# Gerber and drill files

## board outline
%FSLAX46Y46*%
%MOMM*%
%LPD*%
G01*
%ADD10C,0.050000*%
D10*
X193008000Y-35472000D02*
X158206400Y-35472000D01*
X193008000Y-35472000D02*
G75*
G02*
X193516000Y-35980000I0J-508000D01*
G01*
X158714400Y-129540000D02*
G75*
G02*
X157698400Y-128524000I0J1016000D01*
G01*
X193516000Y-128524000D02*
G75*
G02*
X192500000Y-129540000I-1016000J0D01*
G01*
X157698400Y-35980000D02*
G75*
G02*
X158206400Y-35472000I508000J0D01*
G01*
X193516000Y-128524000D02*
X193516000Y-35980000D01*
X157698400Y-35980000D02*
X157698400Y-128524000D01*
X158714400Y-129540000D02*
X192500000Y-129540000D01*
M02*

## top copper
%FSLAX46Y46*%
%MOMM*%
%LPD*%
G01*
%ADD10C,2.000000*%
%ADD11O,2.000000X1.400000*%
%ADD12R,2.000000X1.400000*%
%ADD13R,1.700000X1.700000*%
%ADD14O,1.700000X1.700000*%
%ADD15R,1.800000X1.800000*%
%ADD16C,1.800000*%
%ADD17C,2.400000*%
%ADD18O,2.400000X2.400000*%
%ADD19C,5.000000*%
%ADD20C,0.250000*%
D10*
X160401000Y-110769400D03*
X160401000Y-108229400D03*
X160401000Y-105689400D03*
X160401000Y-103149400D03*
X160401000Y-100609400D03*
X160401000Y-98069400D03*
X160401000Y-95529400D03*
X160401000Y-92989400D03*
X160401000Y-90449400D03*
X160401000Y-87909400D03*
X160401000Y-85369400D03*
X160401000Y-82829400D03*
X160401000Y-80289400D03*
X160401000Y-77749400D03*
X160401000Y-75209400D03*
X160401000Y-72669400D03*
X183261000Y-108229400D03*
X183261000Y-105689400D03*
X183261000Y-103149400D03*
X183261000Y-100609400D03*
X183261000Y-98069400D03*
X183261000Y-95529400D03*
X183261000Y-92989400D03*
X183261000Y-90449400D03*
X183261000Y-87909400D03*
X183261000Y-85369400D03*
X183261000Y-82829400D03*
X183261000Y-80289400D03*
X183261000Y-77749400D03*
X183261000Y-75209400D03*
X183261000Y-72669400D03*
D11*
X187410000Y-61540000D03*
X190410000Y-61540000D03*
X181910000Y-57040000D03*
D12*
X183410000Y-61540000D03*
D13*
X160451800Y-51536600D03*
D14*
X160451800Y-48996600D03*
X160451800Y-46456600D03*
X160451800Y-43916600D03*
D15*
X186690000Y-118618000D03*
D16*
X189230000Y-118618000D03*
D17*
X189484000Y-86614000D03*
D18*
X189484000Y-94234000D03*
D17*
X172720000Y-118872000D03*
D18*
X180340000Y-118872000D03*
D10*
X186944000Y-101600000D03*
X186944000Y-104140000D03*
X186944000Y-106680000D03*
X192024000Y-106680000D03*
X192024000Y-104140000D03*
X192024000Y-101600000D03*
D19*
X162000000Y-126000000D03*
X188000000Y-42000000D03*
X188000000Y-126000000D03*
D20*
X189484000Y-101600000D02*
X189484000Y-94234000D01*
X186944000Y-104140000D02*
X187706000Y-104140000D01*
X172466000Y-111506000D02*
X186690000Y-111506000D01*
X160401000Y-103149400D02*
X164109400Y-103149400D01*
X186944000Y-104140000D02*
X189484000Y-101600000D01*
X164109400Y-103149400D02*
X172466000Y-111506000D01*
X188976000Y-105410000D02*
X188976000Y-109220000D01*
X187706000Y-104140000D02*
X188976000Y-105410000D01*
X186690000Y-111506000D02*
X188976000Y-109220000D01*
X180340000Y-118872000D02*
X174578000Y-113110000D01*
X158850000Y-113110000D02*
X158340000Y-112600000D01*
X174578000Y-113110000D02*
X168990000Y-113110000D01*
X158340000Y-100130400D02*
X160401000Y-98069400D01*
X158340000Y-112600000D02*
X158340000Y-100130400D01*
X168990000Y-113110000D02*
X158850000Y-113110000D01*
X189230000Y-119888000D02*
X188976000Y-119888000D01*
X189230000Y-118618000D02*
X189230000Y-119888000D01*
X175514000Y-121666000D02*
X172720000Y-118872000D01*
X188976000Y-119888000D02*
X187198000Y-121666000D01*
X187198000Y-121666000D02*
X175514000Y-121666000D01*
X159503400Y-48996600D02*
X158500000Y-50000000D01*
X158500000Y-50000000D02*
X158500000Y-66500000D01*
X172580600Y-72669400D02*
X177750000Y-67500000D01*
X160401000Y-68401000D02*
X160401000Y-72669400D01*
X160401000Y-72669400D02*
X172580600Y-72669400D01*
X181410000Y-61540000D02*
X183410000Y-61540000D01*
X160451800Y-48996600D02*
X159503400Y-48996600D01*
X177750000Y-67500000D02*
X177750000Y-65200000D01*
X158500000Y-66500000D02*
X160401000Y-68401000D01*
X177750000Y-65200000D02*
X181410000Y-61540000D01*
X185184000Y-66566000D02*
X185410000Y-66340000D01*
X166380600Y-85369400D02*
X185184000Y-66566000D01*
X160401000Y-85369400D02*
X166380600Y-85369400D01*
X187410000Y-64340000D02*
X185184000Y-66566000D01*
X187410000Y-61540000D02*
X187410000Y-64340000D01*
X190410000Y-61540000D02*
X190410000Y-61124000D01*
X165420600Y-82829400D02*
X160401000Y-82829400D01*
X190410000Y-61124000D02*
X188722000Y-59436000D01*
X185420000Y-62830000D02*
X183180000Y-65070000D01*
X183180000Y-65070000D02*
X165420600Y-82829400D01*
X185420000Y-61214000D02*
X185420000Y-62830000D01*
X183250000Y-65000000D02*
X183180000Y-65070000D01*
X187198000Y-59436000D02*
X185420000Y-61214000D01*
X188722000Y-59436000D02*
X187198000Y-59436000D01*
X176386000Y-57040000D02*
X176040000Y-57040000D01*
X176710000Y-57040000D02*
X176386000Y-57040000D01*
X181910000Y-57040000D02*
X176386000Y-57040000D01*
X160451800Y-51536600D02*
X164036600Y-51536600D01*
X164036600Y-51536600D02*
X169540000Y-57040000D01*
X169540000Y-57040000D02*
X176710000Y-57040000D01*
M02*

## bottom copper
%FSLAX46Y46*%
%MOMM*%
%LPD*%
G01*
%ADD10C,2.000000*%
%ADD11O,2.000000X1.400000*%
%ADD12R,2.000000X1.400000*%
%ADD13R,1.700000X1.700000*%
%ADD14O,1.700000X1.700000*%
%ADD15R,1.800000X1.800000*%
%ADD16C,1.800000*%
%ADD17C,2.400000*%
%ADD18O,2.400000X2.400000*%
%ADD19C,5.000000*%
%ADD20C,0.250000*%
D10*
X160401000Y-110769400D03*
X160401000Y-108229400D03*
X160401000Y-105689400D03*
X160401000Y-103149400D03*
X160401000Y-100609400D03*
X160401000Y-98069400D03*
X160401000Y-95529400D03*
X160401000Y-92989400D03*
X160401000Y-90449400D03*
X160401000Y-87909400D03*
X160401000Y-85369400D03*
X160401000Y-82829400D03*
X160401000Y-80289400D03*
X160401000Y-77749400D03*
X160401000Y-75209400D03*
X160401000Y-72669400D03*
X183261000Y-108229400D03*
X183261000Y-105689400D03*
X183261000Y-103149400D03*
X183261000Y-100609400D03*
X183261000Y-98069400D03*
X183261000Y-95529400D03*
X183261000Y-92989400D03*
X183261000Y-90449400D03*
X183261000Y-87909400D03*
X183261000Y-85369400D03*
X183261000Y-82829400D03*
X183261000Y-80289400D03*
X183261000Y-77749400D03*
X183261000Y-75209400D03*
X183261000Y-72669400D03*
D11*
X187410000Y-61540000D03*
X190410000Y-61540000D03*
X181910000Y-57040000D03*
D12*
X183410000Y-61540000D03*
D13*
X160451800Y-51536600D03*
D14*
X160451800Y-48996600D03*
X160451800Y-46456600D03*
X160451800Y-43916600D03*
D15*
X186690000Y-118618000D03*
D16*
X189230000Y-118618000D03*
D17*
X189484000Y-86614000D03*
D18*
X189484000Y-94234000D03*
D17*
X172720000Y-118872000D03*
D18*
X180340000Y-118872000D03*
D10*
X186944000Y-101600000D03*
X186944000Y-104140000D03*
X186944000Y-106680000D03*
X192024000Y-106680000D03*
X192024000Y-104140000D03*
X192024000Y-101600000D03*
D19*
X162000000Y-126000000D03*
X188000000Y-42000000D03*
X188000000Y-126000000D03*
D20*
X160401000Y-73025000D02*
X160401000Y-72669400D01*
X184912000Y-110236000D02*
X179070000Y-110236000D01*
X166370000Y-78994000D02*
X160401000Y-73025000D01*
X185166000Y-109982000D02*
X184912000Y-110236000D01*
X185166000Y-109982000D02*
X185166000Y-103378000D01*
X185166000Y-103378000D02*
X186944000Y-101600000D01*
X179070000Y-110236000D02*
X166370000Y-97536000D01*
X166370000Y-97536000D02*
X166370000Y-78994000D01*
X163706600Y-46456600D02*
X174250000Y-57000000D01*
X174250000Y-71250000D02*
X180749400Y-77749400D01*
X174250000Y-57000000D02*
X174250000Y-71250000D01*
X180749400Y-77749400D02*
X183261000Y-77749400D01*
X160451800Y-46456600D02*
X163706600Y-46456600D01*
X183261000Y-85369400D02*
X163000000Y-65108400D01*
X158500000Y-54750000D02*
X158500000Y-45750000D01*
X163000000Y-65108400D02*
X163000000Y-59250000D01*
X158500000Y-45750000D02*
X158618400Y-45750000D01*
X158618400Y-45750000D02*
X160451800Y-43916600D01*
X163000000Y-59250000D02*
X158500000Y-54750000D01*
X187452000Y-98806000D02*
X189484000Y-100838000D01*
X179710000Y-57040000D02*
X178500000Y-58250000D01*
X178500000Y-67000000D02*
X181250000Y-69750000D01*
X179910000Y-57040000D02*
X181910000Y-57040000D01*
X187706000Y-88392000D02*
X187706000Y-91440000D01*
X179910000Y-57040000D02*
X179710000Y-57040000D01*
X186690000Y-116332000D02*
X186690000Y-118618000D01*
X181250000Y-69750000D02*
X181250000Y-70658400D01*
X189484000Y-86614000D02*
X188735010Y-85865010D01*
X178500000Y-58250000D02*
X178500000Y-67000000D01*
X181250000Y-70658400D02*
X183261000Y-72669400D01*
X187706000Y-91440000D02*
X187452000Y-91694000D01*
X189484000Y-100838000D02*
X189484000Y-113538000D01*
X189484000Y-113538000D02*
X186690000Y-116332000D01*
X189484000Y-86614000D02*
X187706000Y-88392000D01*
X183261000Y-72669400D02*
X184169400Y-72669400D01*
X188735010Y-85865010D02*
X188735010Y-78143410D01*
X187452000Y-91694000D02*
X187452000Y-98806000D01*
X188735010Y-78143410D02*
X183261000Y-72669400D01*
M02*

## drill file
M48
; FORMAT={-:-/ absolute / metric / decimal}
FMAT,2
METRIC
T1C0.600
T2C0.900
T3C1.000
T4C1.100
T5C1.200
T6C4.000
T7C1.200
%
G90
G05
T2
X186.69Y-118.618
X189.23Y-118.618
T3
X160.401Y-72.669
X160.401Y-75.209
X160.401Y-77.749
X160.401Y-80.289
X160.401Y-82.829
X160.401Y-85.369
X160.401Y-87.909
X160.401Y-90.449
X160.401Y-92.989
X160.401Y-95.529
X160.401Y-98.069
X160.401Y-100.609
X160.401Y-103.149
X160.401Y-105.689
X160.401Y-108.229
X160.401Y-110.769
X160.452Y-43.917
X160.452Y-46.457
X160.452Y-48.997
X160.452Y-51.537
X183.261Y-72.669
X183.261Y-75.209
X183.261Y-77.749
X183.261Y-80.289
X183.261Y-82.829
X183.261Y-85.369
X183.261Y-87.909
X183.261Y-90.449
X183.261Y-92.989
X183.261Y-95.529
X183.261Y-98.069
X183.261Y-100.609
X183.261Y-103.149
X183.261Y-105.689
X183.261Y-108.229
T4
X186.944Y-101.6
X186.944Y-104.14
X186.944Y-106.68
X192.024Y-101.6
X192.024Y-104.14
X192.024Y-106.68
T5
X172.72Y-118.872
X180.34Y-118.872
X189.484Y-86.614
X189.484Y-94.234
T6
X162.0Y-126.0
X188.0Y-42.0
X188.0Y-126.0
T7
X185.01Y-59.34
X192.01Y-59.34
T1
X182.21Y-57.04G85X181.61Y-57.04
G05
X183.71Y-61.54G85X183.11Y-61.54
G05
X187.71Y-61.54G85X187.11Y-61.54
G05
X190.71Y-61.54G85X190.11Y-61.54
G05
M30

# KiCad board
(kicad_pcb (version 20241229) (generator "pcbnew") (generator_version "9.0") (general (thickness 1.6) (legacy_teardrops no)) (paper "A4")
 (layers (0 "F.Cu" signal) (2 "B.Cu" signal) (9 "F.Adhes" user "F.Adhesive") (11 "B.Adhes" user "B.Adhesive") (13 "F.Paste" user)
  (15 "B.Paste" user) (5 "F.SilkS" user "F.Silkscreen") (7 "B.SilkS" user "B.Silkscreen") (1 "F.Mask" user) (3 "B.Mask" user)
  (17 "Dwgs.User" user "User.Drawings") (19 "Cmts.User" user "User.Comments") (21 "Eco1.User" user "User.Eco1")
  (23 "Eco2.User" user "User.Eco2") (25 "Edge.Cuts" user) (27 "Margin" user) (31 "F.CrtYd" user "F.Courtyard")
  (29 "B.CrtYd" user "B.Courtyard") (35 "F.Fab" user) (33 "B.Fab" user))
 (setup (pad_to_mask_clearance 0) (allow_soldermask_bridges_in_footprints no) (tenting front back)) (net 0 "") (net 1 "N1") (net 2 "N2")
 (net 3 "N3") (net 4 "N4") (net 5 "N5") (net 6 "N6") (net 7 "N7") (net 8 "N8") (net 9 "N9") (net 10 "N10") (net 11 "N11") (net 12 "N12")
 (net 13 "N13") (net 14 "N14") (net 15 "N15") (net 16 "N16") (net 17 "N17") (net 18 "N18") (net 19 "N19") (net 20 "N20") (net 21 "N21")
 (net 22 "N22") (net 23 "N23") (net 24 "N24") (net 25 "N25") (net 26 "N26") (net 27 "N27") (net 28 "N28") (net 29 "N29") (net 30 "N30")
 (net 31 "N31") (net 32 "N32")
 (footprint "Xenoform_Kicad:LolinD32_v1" (layer "F.Cu") (at 170.561 90.4494 90)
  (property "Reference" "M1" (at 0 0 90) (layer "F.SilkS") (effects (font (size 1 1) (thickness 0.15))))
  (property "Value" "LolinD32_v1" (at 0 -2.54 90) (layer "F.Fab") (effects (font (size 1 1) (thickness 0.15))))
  (pad "1" thru_hole circle (at -20.32 -10.16 90) (size 2 2) (drill 1) (layers "*.Cu" "*.Mask") (remove_unused_layers no) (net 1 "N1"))
  (pad "2" thru_hole circle (at -17.78 -10.16 90) (size 2 2) (drill 1) (layers "*.Cu" "*.Mask") (remove_unused_layers no) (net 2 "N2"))
  (pad "3" thru_hole circle (at -15.24 -10.16 90) (size 2 2) (drill 1) (layers "*.Cu" "*.Mask") (remove_unused_layers no) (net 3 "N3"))
  (pad "4" thru_hole circle (at -12.7 -10.16 90) (size 2 2) (drill 1) (layers "*.Cu" "*.Mask") (remove_unused_layers no) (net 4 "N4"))
  (pad "5" thru_hole circle (at -10.16 -10.16 90) (size 2 2) (drill 1) (layers "*.Cu" "*.Mask") (remove_unused_layers no) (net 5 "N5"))
  (pad "6" thru_hole circle (at -7.62 -10.16 90) (size 2 2) (drill 1) (layers "*.Cu" "*.Mask") (remove_unused_layers no) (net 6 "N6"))
  (pad "7" thru_hole circle (at -5.08 -10.16 90) (size 2 2) (drill 1) (layers "*.Cu" "*.Mask") (remove_unused_layers no) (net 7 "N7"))
  (pad "8" thru_hole circle (at -2.54 -10.16 90) (size 2 2) (drill 1) (layers "*.Cu" "*.Mask") (remove_unused_layers no) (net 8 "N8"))
  (pad "9" thru_hole circle (at 0 -10.16 90) (size 2 2) (drill 1) (layers "*.Cu" "*.Mask") (remove_unused_layers no) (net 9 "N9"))
  (pad "10" thru_hole circle (at 2.54 -10.16 90) (size 2 2) (drill 1) (layers "*.Cu" "*.Mask") (remove_unused_layers no) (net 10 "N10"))
  (pad "11" thru_hole circle (at 5.08 -10.16 90) (size 2 2) (drill 1) (layers "*.Cu" "*.Mask") (remove_unused_layers no) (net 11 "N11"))
  (pad "12" thru_hole circle (at 7.62 -10.16 90) (size 2 2) (drill 1) (layers "*.Cu" "*.Mask") (remove_unused_layers no) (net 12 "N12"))
  (pad "13" thru_hole circle (at 10.16 -10.16 90) (size 2 2) (drill 1) (layers "*.Cu" "*.Mask") (remove_unused_layers no) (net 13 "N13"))
  (pad "14" thru_hole circle (at 12.7 -10.16 90) (size 2 2) (drill 1) (layers "*.Cu" "*.Mask") (remove_unused_layers no) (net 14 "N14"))
  (pad "15" thru_hole circle (at 15.24 -10.16 90) (size 2 2) (drill 1) (layers "*.Cu" "*.Mask") (remove_unused_layers no) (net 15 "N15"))
  (pad "16" thru_hole circle (at 17.78 -10.16 90) (size 2 2) (drill 1) (layers "*.Cu" "*.Mask") (remove_unused_layers no) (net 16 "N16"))
  (pad "18" thru_hole circle (at -17.78 12.7 90) (size 2 2) (drill 1) (layers "*.Cu" "*.Mask") (remove_unused_layers no) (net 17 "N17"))
  (pad "19" thru_hole circle (at -15.24 12.7 90) (size 2 2) (drill 1) (layers "*.Cu" "*.Mask") (remove_unused_layers no) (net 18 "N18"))
  (pad "20" thru_hole circle (at -12.7 12.7 90) (size 2 2) (drill 1) (layers "*.Cu" "*.Mask") (remove_unused_layers no) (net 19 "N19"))
  (pad "21" thru_hole circle (at -10.16 12.7 90) (size 2 2) (drill 1) (layers "*.Cu" "*.Mask") (remove_unused_layers no) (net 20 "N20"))
  (pad "22" thru_hole circle (at -7.62 12.7 90) (size 2 2) (drill 1) (layers "*.Cu" "*.Mask") (remove_unused_layers no) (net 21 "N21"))
  (pad "23" thru_hole circle (at -5.08 12.7 90) (size 2 2) (drill 1) (layers "*.Cu" "*.Mask") (remove_unused_layers no) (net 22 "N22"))
  (pad "24" thru_hole circle (at -2.54 12.7 90) (size 2 2) (drill 1) (layers "*.Cu" "*.Mask") (remove_unused_layers no) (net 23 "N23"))
  (pad "25" thru_hole circle (at 0 12.7 90) (size 2 2) (drill 1) (layers "*.Cu" "*.Mask") (remove_unused_layers no) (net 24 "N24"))
  (pad "26" thru_hole circle (at 2.54 12.7 90) (size 2 2) (drill 1) (layers "*.Cu" "*.Mask") (remove_unused_layers no) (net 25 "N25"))
  (pad "27" thru_hole circle (at 5.08 12.7 90) (size 2 2) (drill 1) (layers "*.Cu" "*.Mask") (remove_unused_layers no) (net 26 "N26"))
  (pad "28" thru_hole circle (at 7.62 12.7 90) (size 2 2) (drill 1) (layers "*.Cu" "*.Mask") (remove_unused_layers no) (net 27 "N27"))
  (pad "29" thru_hole circle (at 10.16 12.7 90) (size 2 2) (drill 1) (layers "*.Cu" "*.Mask") (remove_unused_layers no) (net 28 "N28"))
  (pad "30" thru_hole circle (at 12.7 12.7 90) (size 2 2) (drill 1) (layers "*.Cu" "*.Mask") (remove_unused_layers no) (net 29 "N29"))
  (pad "31" thru_hole circle (at 15.24 12.7 90) (size 2 2) (drill 1) (layers "*.Cu" "*.Mask") (remove_unused_layers no) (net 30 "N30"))
  (pad "32" thru_hole circle (at 17.78 12.7 90) (size 2 2) (drill 1) (layers "*.Cu" "*.Mask") (remove_unused_layers no) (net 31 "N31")))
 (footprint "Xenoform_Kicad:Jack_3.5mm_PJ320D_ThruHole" (layer "F.Cu") (at 183.41 57.04 -90)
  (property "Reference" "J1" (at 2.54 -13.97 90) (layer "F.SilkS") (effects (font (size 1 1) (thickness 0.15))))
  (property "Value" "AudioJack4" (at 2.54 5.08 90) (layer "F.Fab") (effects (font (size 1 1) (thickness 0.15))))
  (pad "" np_thru_hole circle (at 2.3 -8.6 180) (size 1.2 1.2) (drill 1.2) (layers "*.Cu" "*.Mask"))
  (pad "" np_thru_hole circle (at 2.3 -1.6 180) (size 1.2 1.2) (drill 1.2) (layers "*.Cu" "*.Mask"))
  (pad "R1" thru_hole oval (at 4.5 -4 180) (size 2 1.4) (drill oval 1.2 0.6) (layers "*.Cu" "*.Mask") (remove_unused_layers no)
   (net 11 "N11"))
  (pad "R2" thru_hole oval (at 4.5 -7 180) (size 2 1.4) (drill oval 1.2 0.6) (layers "*.Cu" "*.Mask") (remove_unused_layers no)
   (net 12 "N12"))
  (pad "S" thru_hole oval (at 0 1.5 180) (size 2 1.4) (drill oval 1.2 0.6) (layers "*.Cu" "*.Mask") (remove_unused_layers no) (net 31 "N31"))
  (pad "T" thru_hole rect (at 4.5 0 180) (size 2 1.4) (drill oval 1.2 0.6) (layers "*.Cu" "*.Mask") (remove_unused_layers no) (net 16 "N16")))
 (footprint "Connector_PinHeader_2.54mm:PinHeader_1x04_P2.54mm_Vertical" (layer "F.Cu") (at 160.4518 51.5366 180)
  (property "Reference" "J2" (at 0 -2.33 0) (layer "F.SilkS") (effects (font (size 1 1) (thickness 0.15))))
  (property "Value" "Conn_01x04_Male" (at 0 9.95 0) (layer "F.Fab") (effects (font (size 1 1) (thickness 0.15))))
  (pad "1" thru_hole rect (at 0 0 180) (size 1.7 1.7) (drill 1) (layers "*.Cu" "*.Mask") (remove_unused_layers no) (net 31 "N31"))
  (pad "2" thru_hole oval (at 0 2.54 180) (size 1.7 1.7) (drill 1) (layers "*.Cu" "*.Mask") (remove_unused_layers no) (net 16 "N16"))
  (pad "3" thru_hole oval (at 0 5.08 180) (size 1.7 1.7) (drill 1) (layers "*.Cu" "*.Mask") (remove_unused_layers no) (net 29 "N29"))
  (pad "4" thru_hole oval (at 0 7.62 180) (size 1.7 1.7) (drill 1) (layers "*.Cu" "*.Mask") (remove_unused_layers no) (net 26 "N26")))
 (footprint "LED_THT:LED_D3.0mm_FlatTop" (layer "F.Cu") (at 186.69 118.618)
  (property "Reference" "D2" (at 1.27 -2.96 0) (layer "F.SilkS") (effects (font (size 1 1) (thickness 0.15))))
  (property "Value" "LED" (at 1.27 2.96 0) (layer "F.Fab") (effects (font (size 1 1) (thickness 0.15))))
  (pad "1" thru_hole rect (at 0 0) (size 1.8 1.8) (drill 0.9) (layers "*.Cu" "*.Mask") (remove_unused_layers no) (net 31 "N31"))
  (pad "2" thru_hole circle (at 2.54 0) (size 1.8 1.8) (drill 0.9) (layers "*.Cu" "*.Mask") (remove_unused_layers no) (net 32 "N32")))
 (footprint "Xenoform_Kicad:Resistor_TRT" (layer "F.Cu") (at 189.484 86.614 -90)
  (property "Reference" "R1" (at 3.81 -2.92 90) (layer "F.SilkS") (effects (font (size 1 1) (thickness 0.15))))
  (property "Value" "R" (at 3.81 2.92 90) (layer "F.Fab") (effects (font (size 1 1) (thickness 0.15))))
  (pad "1" thru_hole circle (at 0 0 270) (size 2.4 2.4) (drill 1.2) (layers "*.Cu" "*.Mask") (remove_unused_layers no) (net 31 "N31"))
  (pad "2" thru_hole oval (at 7.62 0 270) (size 2.4 2.4) (drill 1.2) (layers "*.Cu" "*.Mask") (remove_unused_layers no) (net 4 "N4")))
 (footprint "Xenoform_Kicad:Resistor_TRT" (layer "F.Cu") (at 172.72 118.872)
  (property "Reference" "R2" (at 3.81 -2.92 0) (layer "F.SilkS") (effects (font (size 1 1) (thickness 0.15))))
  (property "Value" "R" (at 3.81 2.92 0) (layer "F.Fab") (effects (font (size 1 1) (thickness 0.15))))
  (pad "1" thru_hole circle (at 0 0) (size 2.4 2.4) (drill 1.2) (layers "*.Cu" "*.Mask") (remove_unused_layers no) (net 32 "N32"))
  (pad "2" thru_hole oval (at 7.62 0) (size 2.4 2.4) (drill 1.2) (layers "*.Cu" "*.Mask") (remove_unused_layers no) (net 6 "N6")))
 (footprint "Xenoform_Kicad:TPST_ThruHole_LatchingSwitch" (layer "F.Cu") (at 189.484 104.14)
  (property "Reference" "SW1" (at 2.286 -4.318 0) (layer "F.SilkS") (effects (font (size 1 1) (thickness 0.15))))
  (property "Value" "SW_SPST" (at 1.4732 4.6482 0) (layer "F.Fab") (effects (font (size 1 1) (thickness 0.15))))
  (pad "1" thru_hole circle (at -2.54 -2.54 90) (size 2 2) (drill 1.1) (layers "*.Cu" "*.Mask") (remove_unused_layers no) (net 16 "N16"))
  (pad "2" thru_hole circle (at -2.54 0 90) (size 2 2) (drill 1.1) (layers "*.Cu" "*.Mask") (remove_unused_layers no) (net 4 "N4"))
  (pad "3" thru_hole circle (at -2.54 2.54 90) (size 2 2) (drill 1.1) (layers "*.Cu" "*.Mask") (remove_unused_layers no))
  (pad "4" thru_hole circle (at 2.54 2.54 90) (size 2 2) (drill 1.1) (layers "*.Cu" "*.Mask") (remove_unused_layers no))
  (pad "5" thru_hole circle (at 2.54 0 90) (size 2 2) (drill 1.1) (layers "*.Cu" "*.Mask") (remove_unused_layers no))
  (pad "6" thru_hole circle (at 2.54 -2.54 90) (size 2 2) (drill 1.1) (layers "*.Cu" "*.Mask") (remove_unused_layers no)))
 (gr_line (start 193.008 35.472) (end 158.2064 35.472) (stroke (width 0.05) (type solid)) (layer "Edge.Cuts"))
 (gr_arc (start 193.008 35.472) (mid 193.36721 35.62079) (end 193.516 35.98) (stroke (width 0.05) (type solid)) (layer "Edge.Cuts"))
 (gr_arc (start 158.7144 129.54) (mid 157.99598 129.24242) (end 157.6984 128.524) (stroke (width 0.05) (type solid)) (layer "Edge.Cuts"))
 (gr_arc (start 193.516 128.524) (mid 193.21842 129.24242) (end 192.5 129.54) (stroke (width 0.05) (type solid)) (layer "Edge.Cuts"))
 (gr_arc (start 157.6984 35.98) (mid 157.84719 35.62079) (end 158.2064 35.472) (stroke (width 0.05) (type solid)) (layer "Edge.Cuts"))
 (gr_line (start 193.516 128.524) (end 193.516 35.98) (stroke (width 0.05) (type solid)) (layer "Edge.Cuts"))
 (gr_line (start 157.6984 35.98) (end 157.6984 128.524) (stroke (width 0.05) (type solid)) (layer "Edge.Cuts"))
 (gr_line (start 158.7144 129.54) (end 192.5 129.54) (stroke (width 0.05) (type solid)) (layer "Edge.Cuts"))
 (via (at 162 126) (size 5) (drill 4) (layers "F.Cu" "B.Cu") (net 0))
 (via (at 188 42) (size 5) (drill 4) (layers "F.Cu" "B.Cu") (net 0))
 (via (at 188 126) (size 5) (drill 4) (layers "F.Cu" "B.Cu") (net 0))
 (segment (start 189.484 101.6) (end 189.484 94.234) (width 0.25) (layer "F.Cu") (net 4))
 (segment (start 186.944 104.14) (end 187.706 104.14) (width 0.25) (layer "F.Cu") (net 4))
 (segment (start 172.466 111.506) (end 186.69 111.506) (width 0.25) (layer "F.Cu") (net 4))
 (segment (start 160.401 103.1494) (end 164.1094 103.1494) (width 0.25) (layer "F.Cu") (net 4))
 (segment (start 186.944 104.14) (end 189.484 101.6) (width 0.25) (layer "F.Cu") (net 4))
 (segment (start 164.1094 103.1494) (end 172.466 111.506) (width 0.25) (layer "F.Cu") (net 4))
 (segment (start 188.976 105.41) (end 188.976 109.22) (width 0.25) (layer "F.Cu") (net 4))
 (segment (start 187.706 104.14) (end 188.976 105.41) (width 0.25) (layer "F.Cu") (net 4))
 (segment (start 186.69 111.506) (end 188.976 109.22) (width 0.25) (layer "F.Cu") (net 4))
 (segment (start 180.34 118.872) (end 174.578 113.11) (width 0.25) (layer "F.Cu") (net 6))
 (segment (start 158.85 113.11) (end 158.34 112.6) (width 0.25) (layer "F.Cu") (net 6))
 (segment (start 174.578 113.11) (end 168.99 113.11) (width 0.25) (layer "F.Cu") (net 6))
 (segment (start 158.34 100.1304) (end 160.401 98.0694) (width 0.25) (layer "F.Cu") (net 6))
 (segment (start 158.34 112.6) (end 158.34 100.1304) (width 0.25) (layer "F.Cu") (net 6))
 (segment (start 168.99 113.11) (end 158.85 113.11) (width 0.25) (layer "F.Cu") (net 6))
 (segment (start 189.23 119.888) (end 188.976 119.888) (width 0.25) (layer "F.Cu") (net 32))
 (segment (start 189.23 118.618) (end 189.23 119.888) (width 0.25) (layer "F.Cu") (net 32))
 (segment (start 175.514 121.666) (end 172.72 118.872) (width 0.25) (layer "F.Cu") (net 32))
 (segment (start 188.976 119.888) (end 187.198 121.666) (width 0.25) (layer "F.Cu") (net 32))
 (segment (start 187.198 121.666) (end 175.514 121.666) (width 0.25) (layer "F.Cu") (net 32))
 (segment (start 159.5034 48.9966) (end 158.5 50) (width 0.25) (layer "F.Cu") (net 16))
 (segment (start 158.5 50) (end 158.5 66.5) (width 0.25) (layer "F.Cu") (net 16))
 (segment (start 172.5806 72.6694) (end 177.75 67.5) (width 0.25) (layer "F.Cu") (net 16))
 (segment (start 160.401 68.401) (end 160.401 72.6694) (width 0.25) (layer "F.Cu") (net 16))
 (segment (start 160.401 72.6694) (end 172.5806 72.6694) (width 0.25) (layer "F.Cu") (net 16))
 (segment (start 181.41 61.54) (end 183.41 61.54) (width 0.25) (layer "F.Cu") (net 16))
 (segment (start 160.4518 48.9966) (end 159.5034 48.9966) (width 0.25) (layer "F.Cu") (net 16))
 (segment (start 177.75 67.5) (end 177.75 65.2) (width 0.25) (layer "F.Cu") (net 16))
 (segment (start 158.5 66.5) (end 160.401 68.401) (width 0.25) (layer "F.Cu") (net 16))
 (segment (start 177.75 65.2) (end 181.41 61.54) (width 0.25) (layer "F.Cu") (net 16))
 (segment (start 160.401 73.025) (end 160.401 72.6694) (width 0.25) (layer "B.Cu") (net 16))
 (segment (start 184.912 110.236) (end 179.07 110.236) (width 0.25) (layer "B.Cu") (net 16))
 (segment (start 166.37 78.994) (end 160.401 73.025) (width 0.25) (layer "B.Cu") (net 16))
 (segment (start 185.166 109.982) (end 184.912 110.236) (width 0.25) (layer "B.Cu") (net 16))
 (segment (start 185.166 109.982) (end 185.166 103.378) (width 0.25) (layer "B.Cu") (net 16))
 (segment (start 185.166 103.378) (end 186.944 101.6) (width 0.25) (layer "B.Cu") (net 16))
 (segment (start 179.07 110.236) (end 166.37 97.536) (width 0.25) (layer "B.Cu") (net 16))
 (segment (start 166.37 97.536) (end 166.37 78.994) (width 0.25) (layer "B.Cu") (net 16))
 (segment (start 185.184 66.566) (end 185.41 66.34) (width 0.25) (layer "F.Cu") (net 11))
 (segment (start 166.3806 85.3694) (end 185.184 66.566) (width 0.25) (layer "F.Cu") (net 11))
 (segment (start 160.401 85.3694) (end 166.3806 85.3694) (width 0.25) (layer "F.Cu") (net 11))
 (segment (start 187.41 64.34) (end 185.184 66.566) (width 0.25) (layer "F.Cu") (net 11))
 (segment (start 187.41 61.54) (end 187.41 64.34) (width 0.25) (layer "F.Cu") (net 11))
 (segment (start 190.41 61.54) (end 190.41 61.124) (width 0.25) (layer "F.Cu") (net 12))
 (segment (start 165.4206 82.8294) (end 160.401 82.8294) (width 0.25) (layer "F.Cu") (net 12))
 (segment (start 190.41 61.124) (end 188.722 59.436) (width 0.25) (layer "F.Cu") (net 12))
 (segment (start 185.42 62.83) (end 183.18 65.07) (width 0.25) (layer "F.Cu") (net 12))
 (segment (start 183.18 65.07) (end 165.4206 82.8294) (width 0.25) (layer "F.Cu") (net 12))
 (segment (start 185.42 61.214) (end 185.42 62.83) (width 0.25) (layer "F.Cu") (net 12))
 (segment (start 183.25 65) (end 183.18 65.07) (width 0.25) (layer "F.Cu") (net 12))
 (segment (start 187.198 59.436) (end 185.42 61.214) (width 0.25) (layer "F.Cu") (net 12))
 (segment (start 188.722 59.436) (end 187.198 59.436) (width 0.25) (layer "F.Cu") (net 12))
 (segment (start 163.7066 46.4566) (end 174.25 57) (width 0.25) (layer "B.Cu") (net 29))
 (segment (start 174.25 71.25) (end 180.7494 77.7494) (width 0.25) (layer "B.Cu") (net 29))
 (segment (start 174.25 57) (end 174.25 71.25) (width 0.25) (layer "B.Cu") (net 29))
 (segment (start 180.7494 77.7494) (end 183.261 77.7494) (width 0.25) (layer "B.Cu") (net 29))
 (segment (start 160.4518 46.4566) (end 163.7066 46.4566) (width 0.25) (layer "B.Cu") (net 29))
 (segment (start 183.261 85.3694) (end 163 65.1084) (width 0.25) (layer "B.Cu") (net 26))
 (segment (start 158.5 54.75) (end 158.5 45.75) (width 0.25) (layer "B.Cu") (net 26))
 (segment (start 163 65.1084) (end 163 59.25) (width 0.25) (layer "B.Cu") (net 26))
 (segment (start 158.5 45.75) (end 158.6184 45.75) (width 0.25) (layer "B.Cu") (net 26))
 (segment (start 158.6184 45.75) (end 160.4518 43.9166) (width 0.25) (layer "B.Cu") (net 26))
 (segment (start 163 59.25) (end 158.5 54.75) (width 0.25) (layer "B.Cu") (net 26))
 (segment (start 176.386 57.04) (end 176.04 57.04) (width 0.25) (layer "F.Cu") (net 31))
 (segment (start 176.71 57.04) (end 176.386 57.04) (width 0.25) (layer "F.Cu") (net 31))
 (segment (start 181.91 57.04) (end 176.386 57.04) (width 0.25) (layer "F.Cu") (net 31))
 (segment (start 160.4518 51.5366) (end 164.0366 51.5366) (width 0.25) (layer "F.Cu") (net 31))
 (segment (start 164.0366 51.5366) (end 169.54 57.04) (width 0.25) (layer "F.Cu") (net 31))
 (segment (start 169.54 57.04) (end 176.71 57.04) (width 0.25) (layer "F.Cu") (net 31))
 (segment (start 187.452 98.806) (end 189.484 100.838) (width 0.25) (layer "B.Cu") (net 31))
 (segment (start 179.71 57.04) (end 178.5 58.25) (width 0.25) (layer "B.Cu") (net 31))
 (segment (start 178.5 67) (end 181.25 69.75) (width 0.25) (layer "B.Cu") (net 31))
 (segment (start 179.91 57.04) (end 181.91 57.04) (width 0.25) (layer "B.Cu") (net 31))
 (segment (start 187.706 88.392) (end 187.706 91.44) (width 0.25) (layer "B.Cu") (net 31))
 (segment (start 179.91 57.04) (end 179.71 57.04) (width 0.25) (layer "B.Cu") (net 31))
 (segment (start 186.69 116.332) (end 186.69 118.618) (width 0.25) (layer "B.Cu") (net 31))
 (segment (start 181.25 69.75) (end 181.25 70.6584) (width 0.25) (layer "B.Cu") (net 31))
 (segment (start 189.484 86.614) (end 188.73501 85.86501) (width 0.25) (layer "B.Cu") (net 31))
 (segment (start 178.5 58.25) (end 178.5 67) (width 0.25) (layer "B.Cu") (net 31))
 (segment (start 181.25 70.6584) (end 183.261 72.6694) (width 0.25) (layer "B.Cu") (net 31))
 (segment (start 187.706 91.44) (end 187.452 91.694) (width 0.25) (layer "B.Cu") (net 31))
 (segment (start 189.484 100.838) (end 189.484 113.538) (width 0.25) (layer "B.Cu") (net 31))
 (segment (start 189.484 113.538) (end 186.69 116.332) (width 0.25) (layer "B.Cu") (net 31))
 (segment (start 189.484 86.614) (end 187.706 88.392) (width 0.25) (layer "B.Cu") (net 31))
 (segment (start 183.261 72.6694) (end 184.1694 72.6694) (width 0.25) (layer "B.Cu") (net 31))
 (segment (start 188.73501 85.86501) (end 188.73501 78.14341) (width 0.25) (layer "B.Cu") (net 31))
 (segment (start 187.452 91.694) (end 187.452 98.806) (width 0.25) (layer "B.Cu") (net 31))
 (segment (start 188.73501 78.14341) (end 183.261 72.6694) (width 0.25) (layer "B.Cu") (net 31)))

